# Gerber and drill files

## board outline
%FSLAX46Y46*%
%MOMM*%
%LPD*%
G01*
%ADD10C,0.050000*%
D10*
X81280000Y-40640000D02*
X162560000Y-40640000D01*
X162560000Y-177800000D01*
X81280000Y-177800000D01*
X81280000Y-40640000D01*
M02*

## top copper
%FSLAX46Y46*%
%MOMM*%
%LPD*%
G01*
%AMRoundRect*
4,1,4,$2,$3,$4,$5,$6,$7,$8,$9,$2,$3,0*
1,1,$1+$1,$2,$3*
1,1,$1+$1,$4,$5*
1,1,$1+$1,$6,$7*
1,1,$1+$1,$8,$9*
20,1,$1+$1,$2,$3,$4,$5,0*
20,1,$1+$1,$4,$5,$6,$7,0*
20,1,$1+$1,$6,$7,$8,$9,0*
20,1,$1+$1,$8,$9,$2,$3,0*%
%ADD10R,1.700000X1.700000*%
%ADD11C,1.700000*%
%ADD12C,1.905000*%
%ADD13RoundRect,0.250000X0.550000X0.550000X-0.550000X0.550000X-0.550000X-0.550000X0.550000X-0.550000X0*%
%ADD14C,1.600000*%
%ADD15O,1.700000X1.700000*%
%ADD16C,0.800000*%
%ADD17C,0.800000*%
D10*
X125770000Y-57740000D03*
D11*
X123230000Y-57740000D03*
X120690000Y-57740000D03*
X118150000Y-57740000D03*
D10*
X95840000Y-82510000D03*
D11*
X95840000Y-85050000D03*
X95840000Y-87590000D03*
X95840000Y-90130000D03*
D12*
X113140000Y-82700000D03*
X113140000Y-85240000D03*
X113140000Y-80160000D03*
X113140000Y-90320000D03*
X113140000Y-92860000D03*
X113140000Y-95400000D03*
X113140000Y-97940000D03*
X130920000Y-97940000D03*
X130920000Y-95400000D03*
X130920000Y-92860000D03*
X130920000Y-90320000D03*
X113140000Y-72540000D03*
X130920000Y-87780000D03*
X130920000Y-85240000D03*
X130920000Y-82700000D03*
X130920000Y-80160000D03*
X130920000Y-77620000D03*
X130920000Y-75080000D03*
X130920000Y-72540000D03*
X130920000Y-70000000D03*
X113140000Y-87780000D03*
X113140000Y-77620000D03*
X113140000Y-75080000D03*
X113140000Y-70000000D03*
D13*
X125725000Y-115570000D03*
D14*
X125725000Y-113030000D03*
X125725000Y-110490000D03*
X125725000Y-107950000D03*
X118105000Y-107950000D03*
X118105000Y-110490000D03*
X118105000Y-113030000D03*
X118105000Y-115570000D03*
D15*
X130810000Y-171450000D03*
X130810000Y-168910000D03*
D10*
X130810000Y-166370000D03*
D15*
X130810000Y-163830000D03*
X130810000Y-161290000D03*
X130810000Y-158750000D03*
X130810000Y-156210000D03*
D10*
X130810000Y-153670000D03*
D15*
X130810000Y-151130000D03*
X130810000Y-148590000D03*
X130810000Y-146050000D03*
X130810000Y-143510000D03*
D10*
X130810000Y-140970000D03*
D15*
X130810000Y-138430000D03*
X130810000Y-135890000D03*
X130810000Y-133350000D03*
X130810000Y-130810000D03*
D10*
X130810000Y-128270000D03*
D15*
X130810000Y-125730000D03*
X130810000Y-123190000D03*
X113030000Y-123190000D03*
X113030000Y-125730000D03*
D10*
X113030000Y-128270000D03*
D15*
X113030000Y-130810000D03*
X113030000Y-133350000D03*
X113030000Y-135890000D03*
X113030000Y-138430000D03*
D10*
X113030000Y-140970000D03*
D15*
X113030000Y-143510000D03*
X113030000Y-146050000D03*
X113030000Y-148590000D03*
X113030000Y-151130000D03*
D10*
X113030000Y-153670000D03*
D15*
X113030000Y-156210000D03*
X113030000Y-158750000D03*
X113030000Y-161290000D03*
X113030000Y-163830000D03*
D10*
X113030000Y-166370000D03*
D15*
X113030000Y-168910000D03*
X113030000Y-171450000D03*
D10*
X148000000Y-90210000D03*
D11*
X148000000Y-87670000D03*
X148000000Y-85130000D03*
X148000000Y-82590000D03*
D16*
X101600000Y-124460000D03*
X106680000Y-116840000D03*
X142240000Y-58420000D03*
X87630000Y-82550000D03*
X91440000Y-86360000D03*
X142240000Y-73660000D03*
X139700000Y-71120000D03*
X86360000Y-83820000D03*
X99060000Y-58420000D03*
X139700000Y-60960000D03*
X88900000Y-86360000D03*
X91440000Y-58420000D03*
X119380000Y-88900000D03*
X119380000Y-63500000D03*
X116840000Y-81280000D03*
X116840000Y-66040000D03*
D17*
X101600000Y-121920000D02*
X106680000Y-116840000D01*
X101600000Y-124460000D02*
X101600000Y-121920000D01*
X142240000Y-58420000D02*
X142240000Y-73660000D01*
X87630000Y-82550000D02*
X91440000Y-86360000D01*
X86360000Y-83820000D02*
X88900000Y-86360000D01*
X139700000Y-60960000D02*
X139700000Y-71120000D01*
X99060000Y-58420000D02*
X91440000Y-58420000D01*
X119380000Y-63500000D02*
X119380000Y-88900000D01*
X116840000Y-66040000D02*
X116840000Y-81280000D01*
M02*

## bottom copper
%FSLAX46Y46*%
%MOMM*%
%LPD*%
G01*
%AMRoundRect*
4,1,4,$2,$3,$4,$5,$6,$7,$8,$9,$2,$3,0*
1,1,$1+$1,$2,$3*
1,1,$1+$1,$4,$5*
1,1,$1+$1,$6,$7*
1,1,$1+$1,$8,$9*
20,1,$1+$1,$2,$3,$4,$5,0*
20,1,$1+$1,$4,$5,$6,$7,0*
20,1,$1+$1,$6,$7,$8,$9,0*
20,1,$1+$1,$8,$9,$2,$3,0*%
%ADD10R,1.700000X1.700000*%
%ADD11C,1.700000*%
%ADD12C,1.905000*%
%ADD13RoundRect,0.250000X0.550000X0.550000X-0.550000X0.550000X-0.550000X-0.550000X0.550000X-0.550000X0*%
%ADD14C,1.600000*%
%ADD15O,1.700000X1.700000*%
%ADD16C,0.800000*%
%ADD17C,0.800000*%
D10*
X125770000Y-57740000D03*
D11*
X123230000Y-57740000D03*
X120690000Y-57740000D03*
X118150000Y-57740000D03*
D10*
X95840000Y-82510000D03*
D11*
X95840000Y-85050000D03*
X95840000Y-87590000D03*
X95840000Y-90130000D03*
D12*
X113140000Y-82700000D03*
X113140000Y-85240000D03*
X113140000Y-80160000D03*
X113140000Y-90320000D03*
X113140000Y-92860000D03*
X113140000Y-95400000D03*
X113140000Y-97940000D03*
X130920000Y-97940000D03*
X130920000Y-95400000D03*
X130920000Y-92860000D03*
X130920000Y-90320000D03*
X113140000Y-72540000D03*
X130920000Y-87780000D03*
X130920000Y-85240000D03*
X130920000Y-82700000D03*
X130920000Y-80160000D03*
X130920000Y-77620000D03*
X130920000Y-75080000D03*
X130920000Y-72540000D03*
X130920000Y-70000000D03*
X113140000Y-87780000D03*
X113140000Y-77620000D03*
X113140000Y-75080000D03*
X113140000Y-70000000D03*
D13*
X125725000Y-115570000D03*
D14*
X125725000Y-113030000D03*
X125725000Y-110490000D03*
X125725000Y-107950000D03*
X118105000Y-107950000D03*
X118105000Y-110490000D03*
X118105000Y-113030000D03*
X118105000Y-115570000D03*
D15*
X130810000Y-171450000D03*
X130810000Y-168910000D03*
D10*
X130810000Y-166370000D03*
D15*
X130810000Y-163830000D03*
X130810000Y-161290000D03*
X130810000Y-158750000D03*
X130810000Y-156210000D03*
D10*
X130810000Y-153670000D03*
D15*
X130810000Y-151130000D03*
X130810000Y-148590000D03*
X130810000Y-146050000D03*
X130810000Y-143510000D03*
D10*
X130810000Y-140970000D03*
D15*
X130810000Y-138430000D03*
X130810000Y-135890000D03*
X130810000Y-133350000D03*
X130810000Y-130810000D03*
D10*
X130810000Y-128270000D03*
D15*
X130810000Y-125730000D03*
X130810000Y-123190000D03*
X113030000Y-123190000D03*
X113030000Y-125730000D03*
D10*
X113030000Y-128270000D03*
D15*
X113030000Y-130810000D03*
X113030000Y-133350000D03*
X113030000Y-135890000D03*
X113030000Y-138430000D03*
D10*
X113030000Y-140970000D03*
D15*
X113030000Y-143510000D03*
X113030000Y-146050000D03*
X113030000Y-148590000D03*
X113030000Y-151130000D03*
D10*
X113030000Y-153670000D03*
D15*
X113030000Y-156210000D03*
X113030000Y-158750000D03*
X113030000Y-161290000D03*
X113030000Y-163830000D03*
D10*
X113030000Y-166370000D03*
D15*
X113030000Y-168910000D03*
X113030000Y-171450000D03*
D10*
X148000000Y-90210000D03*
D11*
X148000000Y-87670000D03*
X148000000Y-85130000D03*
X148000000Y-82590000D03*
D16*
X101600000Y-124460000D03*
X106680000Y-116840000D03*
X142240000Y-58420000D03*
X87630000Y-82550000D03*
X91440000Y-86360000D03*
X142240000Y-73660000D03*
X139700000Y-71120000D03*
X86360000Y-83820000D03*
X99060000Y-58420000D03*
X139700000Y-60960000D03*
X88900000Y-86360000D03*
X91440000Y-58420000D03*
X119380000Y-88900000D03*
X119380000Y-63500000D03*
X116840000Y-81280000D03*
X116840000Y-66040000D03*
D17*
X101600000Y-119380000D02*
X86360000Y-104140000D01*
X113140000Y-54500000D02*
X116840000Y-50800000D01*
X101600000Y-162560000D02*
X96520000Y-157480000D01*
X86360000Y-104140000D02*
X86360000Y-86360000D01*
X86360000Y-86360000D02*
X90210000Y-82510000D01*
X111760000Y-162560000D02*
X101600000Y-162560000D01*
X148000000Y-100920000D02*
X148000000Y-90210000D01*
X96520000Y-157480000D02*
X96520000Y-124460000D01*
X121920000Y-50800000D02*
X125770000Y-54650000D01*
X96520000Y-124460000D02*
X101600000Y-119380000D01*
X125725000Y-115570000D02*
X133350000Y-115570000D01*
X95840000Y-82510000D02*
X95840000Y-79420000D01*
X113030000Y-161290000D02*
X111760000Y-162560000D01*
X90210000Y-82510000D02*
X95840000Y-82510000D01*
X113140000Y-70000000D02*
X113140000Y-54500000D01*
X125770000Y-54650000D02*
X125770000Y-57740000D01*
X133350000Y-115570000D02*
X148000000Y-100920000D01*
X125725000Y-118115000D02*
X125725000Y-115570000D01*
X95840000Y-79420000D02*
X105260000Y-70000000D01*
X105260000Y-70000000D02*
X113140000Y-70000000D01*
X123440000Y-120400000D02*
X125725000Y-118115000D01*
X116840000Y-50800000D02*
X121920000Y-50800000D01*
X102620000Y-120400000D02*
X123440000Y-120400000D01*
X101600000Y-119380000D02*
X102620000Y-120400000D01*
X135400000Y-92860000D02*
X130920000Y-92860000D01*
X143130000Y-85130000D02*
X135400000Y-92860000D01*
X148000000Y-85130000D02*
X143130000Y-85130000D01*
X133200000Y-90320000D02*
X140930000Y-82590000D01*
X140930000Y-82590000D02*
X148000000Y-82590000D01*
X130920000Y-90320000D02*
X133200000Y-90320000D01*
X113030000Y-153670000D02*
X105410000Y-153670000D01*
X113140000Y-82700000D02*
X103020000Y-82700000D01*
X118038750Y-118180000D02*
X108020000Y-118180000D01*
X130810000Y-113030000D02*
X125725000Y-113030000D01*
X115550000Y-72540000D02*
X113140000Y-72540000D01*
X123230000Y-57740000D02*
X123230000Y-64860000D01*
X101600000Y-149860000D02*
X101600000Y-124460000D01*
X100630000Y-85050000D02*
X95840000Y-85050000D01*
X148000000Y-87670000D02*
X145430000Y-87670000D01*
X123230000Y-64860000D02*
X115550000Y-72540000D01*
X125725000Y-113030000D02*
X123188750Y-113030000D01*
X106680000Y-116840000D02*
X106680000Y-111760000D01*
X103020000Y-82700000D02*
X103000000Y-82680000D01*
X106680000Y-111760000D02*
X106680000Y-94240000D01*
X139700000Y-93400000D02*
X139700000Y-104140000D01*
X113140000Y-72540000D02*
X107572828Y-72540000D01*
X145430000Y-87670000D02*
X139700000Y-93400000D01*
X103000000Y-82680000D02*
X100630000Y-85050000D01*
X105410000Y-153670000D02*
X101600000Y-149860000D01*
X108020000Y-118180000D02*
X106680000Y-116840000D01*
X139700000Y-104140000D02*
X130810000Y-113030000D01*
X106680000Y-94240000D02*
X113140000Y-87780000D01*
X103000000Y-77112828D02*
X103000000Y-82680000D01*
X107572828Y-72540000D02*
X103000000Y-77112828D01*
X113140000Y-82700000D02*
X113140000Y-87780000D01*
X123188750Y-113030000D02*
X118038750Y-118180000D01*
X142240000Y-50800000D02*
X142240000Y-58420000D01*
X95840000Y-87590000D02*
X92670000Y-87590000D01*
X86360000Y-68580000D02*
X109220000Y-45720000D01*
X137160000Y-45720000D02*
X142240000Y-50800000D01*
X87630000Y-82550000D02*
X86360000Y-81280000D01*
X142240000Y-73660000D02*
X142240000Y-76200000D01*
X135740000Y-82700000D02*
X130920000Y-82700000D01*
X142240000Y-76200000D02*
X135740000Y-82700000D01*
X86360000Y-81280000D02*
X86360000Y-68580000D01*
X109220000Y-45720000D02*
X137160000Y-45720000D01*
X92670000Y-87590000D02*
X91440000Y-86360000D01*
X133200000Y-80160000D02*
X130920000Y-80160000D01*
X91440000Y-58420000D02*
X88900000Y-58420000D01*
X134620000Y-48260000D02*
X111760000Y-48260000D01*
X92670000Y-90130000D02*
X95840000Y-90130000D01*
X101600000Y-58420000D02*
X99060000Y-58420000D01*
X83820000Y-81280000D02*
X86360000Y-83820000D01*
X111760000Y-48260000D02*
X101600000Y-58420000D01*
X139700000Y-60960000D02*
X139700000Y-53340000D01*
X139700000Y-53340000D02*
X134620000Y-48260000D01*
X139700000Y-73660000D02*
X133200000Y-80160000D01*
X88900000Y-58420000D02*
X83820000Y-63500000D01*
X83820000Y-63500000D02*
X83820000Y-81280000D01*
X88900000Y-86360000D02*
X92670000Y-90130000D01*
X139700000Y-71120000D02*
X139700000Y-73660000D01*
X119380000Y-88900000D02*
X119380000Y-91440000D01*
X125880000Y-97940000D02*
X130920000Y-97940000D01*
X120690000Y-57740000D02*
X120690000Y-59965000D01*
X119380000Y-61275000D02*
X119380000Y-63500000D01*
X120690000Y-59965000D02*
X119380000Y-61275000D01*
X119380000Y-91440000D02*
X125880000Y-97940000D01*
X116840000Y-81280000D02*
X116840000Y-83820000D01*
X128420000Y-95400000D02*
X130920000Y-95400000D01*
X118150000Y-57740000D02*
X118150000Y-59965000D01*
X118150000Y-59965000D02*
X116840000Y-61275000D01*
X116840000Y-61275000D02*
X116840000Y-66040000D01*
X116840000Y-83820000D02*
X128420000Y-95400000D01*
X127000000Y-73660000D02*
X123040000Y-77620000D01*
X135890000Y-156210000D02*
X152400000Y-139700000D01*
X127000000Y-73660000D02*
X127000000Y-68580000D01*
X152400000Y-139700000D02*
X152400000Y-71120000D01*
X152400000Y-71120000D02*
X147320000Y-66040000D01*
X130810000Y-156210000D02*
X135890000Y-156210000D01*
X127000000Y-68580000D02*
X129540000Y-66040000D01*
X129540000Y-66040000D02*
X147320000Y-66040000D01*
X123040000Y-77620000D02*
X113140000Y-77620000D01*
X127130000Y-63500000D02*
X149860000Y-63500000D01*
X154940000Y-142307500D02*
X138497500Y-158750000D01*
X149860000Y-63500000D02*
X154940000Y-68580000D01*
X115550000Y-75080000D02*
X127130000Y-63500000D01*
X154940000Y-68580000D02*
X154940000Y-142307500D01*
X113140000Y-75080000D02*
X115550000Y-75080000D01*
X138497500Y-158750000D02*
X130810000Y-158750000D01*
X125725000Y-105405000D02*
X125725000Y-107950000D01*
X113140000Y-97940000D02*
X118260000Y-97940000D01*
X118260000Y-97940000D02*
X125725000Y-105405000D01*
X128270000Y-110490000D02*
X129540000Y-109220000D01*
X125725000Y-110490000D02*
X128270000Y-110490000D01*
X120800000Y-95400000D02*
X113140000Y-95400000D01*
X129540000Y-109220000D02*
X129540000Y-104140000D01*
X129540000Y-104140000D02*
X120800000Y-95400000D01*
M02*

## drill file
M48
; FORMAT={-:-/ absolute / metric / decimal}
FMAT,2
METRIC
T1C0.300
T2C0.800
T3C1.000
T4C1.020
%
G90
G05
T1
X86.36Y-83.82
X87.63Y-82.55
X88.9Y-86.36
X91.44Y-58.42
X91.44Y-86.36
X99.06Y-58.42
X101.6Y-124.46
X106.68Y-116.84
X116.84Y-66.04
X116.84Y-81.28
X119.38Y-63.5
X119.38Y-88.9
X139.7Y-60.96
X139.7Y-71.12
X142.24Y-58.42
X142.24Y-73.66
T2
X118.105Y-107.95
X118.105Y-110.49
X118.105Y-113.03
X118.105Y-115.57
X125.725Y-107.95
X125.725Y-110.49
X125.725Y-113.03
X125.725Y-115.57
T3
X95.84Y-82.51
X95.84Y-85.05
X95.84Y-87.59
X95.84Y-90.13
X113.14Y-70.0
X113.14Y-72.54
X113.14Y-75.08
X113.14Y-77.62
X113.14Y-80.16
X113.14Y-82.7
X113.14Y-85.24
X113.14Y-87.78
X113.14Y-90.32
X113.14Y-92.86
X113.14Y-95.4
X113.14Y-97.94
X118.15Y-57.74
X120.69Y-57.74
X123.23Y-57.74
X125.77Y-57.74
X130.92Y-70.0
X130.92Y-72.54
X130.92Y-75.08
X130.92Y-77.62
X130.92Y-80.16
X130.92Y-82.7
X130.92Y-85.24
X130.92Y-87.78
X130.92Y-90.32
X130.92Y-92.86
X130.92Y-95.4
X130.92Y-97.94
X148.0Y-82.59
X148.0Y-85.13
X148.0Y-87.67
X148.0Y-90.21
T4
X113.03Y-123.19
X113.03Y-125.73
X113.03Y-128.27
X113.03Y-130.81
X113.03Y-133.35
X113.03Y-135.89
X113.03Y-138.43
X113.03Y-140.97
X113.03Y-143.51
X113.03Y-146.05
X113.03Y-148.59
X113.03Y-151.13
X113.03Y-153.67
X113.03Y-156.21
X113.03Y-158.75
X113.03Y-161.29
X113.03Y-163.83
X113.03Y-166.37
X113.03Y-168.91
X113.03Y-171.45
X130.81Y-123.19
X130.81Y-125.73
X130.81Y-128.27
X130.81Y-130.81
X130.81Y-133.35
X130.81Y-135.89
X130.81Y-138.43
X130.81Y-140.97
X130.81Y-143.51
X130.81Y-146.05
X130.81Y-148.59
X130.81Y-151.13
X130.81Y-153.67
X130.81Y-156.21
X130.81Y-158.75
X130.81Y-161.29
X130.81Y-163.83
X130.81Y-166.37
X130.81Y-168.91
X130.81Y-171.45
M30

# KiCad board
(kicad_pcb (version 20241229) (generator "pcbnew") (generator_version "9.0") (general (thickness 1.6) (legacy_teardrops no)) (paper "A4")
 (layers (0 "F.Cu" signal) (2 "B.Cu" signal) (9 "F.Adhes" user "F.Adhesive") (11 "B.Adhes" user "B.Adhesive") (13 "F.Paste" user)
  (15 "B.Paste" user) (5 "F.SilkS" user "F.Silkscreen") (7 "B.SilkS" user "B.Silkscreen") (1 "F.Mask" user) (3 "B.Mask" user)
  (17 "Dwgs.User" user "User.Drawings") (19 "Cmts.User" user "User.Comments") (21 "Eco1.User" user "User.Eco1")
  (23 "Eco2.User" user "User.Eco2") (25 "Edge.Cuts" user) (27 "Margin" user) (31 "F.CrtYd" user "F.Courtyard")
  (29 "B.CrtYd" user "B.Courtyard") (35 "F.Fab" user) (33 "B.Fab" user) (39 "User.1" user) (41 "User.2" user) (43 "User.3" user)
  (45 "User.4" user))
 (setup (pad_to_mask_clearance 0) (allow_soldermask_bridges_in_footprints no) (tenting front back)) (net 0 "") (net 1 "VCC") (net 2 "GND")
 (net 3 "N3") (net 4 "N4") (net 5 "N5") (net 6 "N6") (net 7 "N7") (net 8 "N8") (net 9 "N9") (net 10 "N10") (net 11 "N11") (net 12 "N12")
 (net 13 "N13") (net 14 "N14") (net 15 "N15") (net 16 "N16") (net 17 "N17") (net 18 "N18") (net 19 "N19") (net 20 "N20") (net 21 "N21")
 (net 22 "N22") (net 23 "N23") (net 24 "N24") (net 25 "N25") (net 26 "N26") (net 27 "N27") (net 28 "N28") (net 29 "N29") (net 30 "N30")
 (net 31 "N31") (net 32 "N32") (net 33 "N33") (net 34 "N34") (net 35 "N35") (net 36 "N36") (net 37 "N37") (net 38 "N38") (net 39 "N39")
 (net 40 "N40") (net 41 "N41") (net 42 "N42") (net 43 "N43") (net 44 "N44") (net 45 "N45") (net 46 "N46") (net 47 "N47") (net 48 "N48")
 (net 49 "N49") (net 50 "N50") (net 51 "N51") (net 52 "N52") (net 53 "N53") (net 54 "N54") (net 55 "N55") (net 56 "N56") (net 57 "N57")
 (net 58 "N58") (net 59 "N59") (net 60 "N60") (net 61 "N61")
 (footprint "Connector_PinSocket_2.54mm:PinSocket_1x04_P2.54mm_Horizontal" (layer "F.Cu") (at 125.77 57.74 -90)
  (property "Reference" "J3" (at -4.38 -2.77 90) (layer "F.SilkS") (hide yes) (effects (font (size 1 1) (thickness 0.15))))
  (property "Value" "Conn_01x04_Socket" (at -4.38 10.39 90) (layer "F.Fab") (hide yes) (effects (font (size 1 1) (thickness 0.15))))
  (pad "1" thru_hole rect (at 0 0 270) (size 1.7 1.7) (drill 1) (layers "*.Cu" "*.Mask") (remove_unused_layers no) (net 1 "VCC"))
  (pad "2" thru_hole circle (at 0 2.54 270) (size 1.7 1.7) (drill 1) (layers "*.Cu" "*.Mask") (remove_unused_layers no) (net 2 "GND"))
  (pad "3" thru_hole circle (at 0 5.08 270) (size 1.7 1.7) (drill 1) (layers "*.Cu" "*.Mask") (remove_unused_layers no) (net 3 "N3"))
  (pad "4" thru_hole circle (at 0 7.62 270) (size 1.7 1.7) (drill 1) (layers "*.Cu" "*.Mask") (remove_unused_layers no) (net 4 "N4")))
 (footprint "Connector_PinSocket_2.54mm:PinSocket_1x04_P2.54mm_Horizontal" (layer "F.Cu") (at 95.84 82.51)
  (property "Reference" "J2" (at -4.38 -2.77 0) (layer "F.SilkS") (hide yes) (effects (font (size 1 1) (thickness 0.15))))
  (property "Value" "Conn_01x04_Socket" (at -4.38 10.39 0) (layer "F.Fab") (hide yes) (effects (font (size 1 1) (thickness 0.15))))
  (pad "1" thru_hole rect (at 0 0) (size 1.7 1.7) (drill 1) (layers "*.Cu" "*.Mask") (remove_unused_layers no) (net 1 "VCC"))
  (pad "2" thru_hole circle (at 0 2.54) (size 1.7 1.7) (drill 1) (layers "*.Cu" "*.Mask") (remove_unused_layers no) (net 2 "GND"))
  (pad "3" thru_hole circle (at 0 5.08) (size 1.7 1.7) (drill 1) (layers "*.Cu" "*.Mask") (remove_unused_layers no) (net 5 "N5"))
  (pad "4" thru_hole circle (at 0 7.62) (size 1.7 1.7) (drill 1) (layers "*.Cu" "*.Mask") (remove_unused_layers no) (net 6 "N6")))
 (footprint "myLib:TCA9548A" (layer "F.Cu") (at 121.92 73.82)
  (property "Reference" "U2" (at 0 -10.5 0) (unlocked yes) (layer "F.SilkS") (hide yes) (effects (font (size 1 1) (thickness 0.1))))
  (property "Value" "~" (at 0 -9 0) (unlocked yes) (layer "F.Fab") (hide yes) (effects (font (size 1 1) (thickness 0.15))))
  (pad "1" thru_hole circle (at -8.78 8.88) (size 1.905 1.905) (drill 1) (layers "*.Cu" "*.Mask") (remove_unused_layers no) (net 2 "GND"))
  (pad "2" thru_hole circle (at -8.78 11.42) (size 1.905 1.905) (drill 1) (layers "*.Cu" "*.Mask") (remove_unused_layers no) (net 2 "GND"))
  (pad "3" thru_hole circle (at -8.78 6.34) (size 1.905 1.905) (drill 1) (layers "*.Cu" "*.Mask") (remove_unused_layers no) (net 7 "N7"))
  (pad "4" thru_hole circle (at -8.78 16.5) (size 1.905 1.905) (drill 1) (layers "*.Cu" "*.Mask") (remove_unused_layers no) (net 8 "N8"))
  (pad "5" thru_hole circle (at -8.78 19.04) (size 1.905 1.905) (drill 1) (layers "*.Cu" "*.Mask") (remove_unused_layers no) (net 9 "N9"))
  (pad "6" thru_hole circle (at -8.78 21.58) (size 1.905 1.905) (drill 1) (layers "*.Cu" "*.Mask") (remove_unused_layers no) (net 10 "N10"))
  (pad "7" thru_hole circle (at -8.78 24.12) (size 1.905 1.905) (drill 1) (layers "*.Cu" "*.Mask") (remove_unused_layers no) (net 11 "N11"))
  (pad "8" thru_hole circle (at 9 24.12) (size 1.905 1.905) (drill 1) (layers "*.Cu" "*.Mask") (remove_unused_layers no) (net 3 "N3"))
  (pad "9" thru_hole circle (at 9 21.58) (size 1.905 1.905) (drill 1) (layers "*.Cu" "*.Mask") (remove_unused_layers no) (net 4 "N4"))
  (pad "10" thru_hole circle (at 9 19.04) (size 1.905 1.905) (drill 1) (layers "*.Cu" "*.Mask") (remove_unused_layers no) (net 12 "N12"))
  (pad "11" thru_hole circle (at 9 16.5) (size 1.905 1.905) (drill 1) (layers "*.Cu" "*.Mask") (remove_unused_layers no) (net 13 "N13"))
  (pad "12" thru_hole circle (at -8.78 -1.28) (size 1.905 1.905) (drill 1) (layers "*.Cu" "*.Mask") (remove_unused_layers no) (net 2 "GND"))
  (pad "13" thru_hole circle (at 9 13.96) (size 1.905 1.905) (drill 1) (layers "*.Cu" "*.Mask") (remove_unused_layers no) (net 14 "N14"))
  (pad "14" thru_hole circle (at 9 11.42) (size 1.905 1.905) (drill 1) (layers "*.Cu" "*.Mask") (remove_unused_layers no) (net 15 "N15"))
  (pad "15" thru_hole circle (at 9 8.88) (size 1.905 1.905) (drill 1) (layers "*.Cu" "*.Mask") (remove_unused_layers no) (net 5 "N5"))
  (pad "16" thru_hole circle (at 9 6.34) (size 1.905 1.905) (drill 1) (layers "*.Cu" "*.Mask") (remove_unused_layers no) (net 6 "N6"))
  (pad "17" thru_hole circle (at 9 3.8) (size 1.905 1.905) (drill 1) (layers "*.Cu" "*.Mask") (remove_unused_layers no) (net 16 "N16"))
  (pad "18" thru_hole circle (at 9 1.26) (size 1.905 1.905) (drill 1) (layers "*.Cu" "*.Mask") (remove_unused_layers no) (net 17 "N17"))
  (pad "19" thru_hole circle (at 9 -1.28) (size 1.905 1.905) (drill 1) (layers "*.Cu" "*.Mask") (remove_unused_layers no) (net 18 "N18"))
  (pad "20" thru_hole circle (at 9 -3.82) (size 1.905 1.905) (drill 1) (layers "*.Cu" "*.Mask") (remove_unused_layers no) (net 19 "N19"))
  (pad "21" thru_hole circle (at -8.78 13.96) (size 1.905 1.905) (drill 1) (layers "*.Cu" "*.Mask") (remove_unused_layers no) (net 2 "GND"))
  (pad "22" thru_hole circle (at -8.78 3.8) (size 1.905 1.905) (drill 1) (layers "*.Cu" "*.Mask") (remove_unused_layers no) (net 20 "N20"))
  (pad "23" thru_hole circle (at -8.78 1.26) (size 1.905 1.905) (drill 1) (layers "*.Cu" "*.Mask") (remove_unused_layers no) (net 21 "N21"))
  (pad "24" thru_hole circle (at -8.78 -3.82) (size 1.905 1.905) (drill 1) (layers "*.Cu" "*.Mask") (remove_unused_layers no) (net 1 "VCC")))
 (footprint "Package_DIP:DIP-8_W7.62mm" (layer "F.Cu") (at 125.725 115.57 180)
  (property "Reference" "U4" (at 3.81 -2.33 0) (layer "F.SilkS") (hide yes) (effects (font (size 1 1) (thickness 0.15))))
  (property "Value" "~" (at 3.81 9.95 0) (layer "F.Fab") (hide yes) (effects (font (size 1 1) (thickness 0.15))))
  (pad "1" thru_hole roundrect (at 0 0 180) (size 1.6 1.6) (drill 0.8) (layers "*.Cu" "*.Mask") (remove_unused_layers no)
   (roundrect_rratio 0.15625) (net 1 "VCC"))
  (pad "2" thru_hole circle (at 0 2.54 180) (size 1.6 1.6) (drill 0.8) (layers "*.Cu" "*.Mask") (remove_unused_layers no) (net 2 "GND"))
  (pad "3" thru_hole circle (at 0 5.08 180) (size 1.6 1.6) (drill 0.8) (layers "*.Cu" "*.Mask") (remove_unused_layers no) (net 10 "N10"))
  (pad "4" thru_hole circle (at 0 7.62 180) (size 1.6 1.6) (drill 0.8) (layers "*.Cu" "*.Mask") (remove_unused_layers no) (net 11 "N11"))
  (pad "5" thru_hole circle (at 7.62 7.62 180) (size 1.6 1.6) (drill 0.8) (layers "*.Cu" "*.Mask") (remove_unused_layers no) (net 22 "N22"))
  (pad "6" thru_hole circle (at 7.62 5.08 180) (size 1.6 1.6) (drill 0.8) (layers "*.Cu" "*.Mask") (remove_unused_layers no) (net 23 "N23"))
  (pad "7" thru_hole circle (at 7.62 2.54 180) (size 1.6 1.6) (drill 0.8) (layers "*.Cu" "*.Mask") (remove_unused_layers no) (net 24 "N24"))
  (pad "8" thru_hole circle (at 7.62 0 180) (size 1.6 1.6) (drill 0.8) (layers "*.Cu" "*.Mask") (remove_unused_layers no) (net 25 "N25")))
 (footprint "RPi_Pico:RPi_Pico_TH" (layer "F.Cu") (at 121.92 147.32 180)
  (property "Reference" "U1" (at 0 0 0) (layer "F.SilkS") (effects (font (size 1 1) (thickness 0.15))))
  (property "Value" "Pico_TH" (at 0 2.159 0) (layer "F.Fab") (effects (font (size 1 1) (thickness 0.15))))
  (pad "1" thru_hole oval (at -8.89 -24.13 180) (size 1.7 1.7) (drill 1.02) (layers "*.Cu" "*.Mask") (remove_unused_layers no)
   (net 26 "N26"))
  (pad "2" thru_hole oval (at -8.89 -21.59 180) (size 1.7 1.7) (drill 1.02) (layers "*.Cu" "*.Mask") (remove_unused_layers no)
   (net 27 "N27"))
  (pad "3" thru_hole rect (at -8.89 -19.05 180) (size 1.7 1.7) (drill 1.02) (layers "*.Cu" "*.Mask") (remove_unused_layers no)
   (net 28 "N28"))
  (pad "4" thru_hole oval (at -8.89 -16.51 180) (size 1.7 1.7) (drill 1.02) (layers "*.Cu" "*.Mask") (remove_unused_layers no)
   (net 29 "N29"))
  (pad "5" thru_hole oval (at -8.89 -13.97 180) (size 1.7 1.7) (drill 1.02) (layers "*.Cu" "*.Mask") (remove_unused_layers no)
   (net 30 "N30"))
  (pad "6" thru_hole oval (at -8.89 -11.43 180) (size 1.7 1.7) (drill 1.02) (layers "*.Cu" "*.Mask") (remove_unused_layers no)
   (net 21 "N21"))
  (pad "7" thru_hole oval (at -8.89 -8.89 180) (size 1.7 1.7) (drill 1.02) (layers "*.Cu" "*.Mask") (remove_unused_layers no) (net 20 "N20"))
  (pad "8" thru_hole rect (at -8.89 -6.35 180) (size 1.7 1.7) (drill 1.02) (layers "*.Cu" "*.Mask") (remove_unused_layers no) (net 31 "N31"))
  (pad "9" thru_hole oval (at -8.89 -3.81 180) (size 1.7 1.7) (drill 1.02) (layers "*.Cu" "*.Mask") (remove_unused_layers no) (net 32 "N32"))
  (pad "10" thru_hole oval (at -8.89 -1.27 180) (size 1.7 1.7) (drill 1.02) (layers "*.Cu" "*.Mask") (remove_unused_layers no)
   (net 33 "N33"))
  (pad "11" thru_hole oval (at -8.89 1.27 180) (size 1.7 1.7) (drill 1.02) (layers "*.Cu" "*.Mask") (remove_unused_layers no) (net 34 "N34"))
  (pad "12" thru_hole oval (at -8.89 3.81 180) (size 1.7 1.7) (drill 1.02) (layers "*.Cu" "*.Mask") (remove_unused_layers no) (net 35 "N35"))
  (pad "13" thru_hole rect (at -8.89 6.35 180) (size 1.7 1.7) (drill 1.02) (layers "*.Cu" "*.Mask") (remove_unused_layers no) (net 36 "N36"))
  (pad "14" thru_hole oval (at -8.89 8.89 180) (size 1.7 1.7) (drill 1.02) (layers "*.Cu" "*.Mask") (remove_unused_layers no) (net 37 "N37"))
  (pad "15" thru_hole oval (at -8.89 11.43 180) (size 1.7 1.7) (drill 1.02) (layers "*.Cu" "*.Mask") (remove_unused_layers no)
   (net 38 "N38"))
  (pad "16" thru_hole oval (at -8.89 13.97 180) (size 1.7 1.7) (drill 1.02) (layers "*.Cu" "*.Mask") (remove_unused_layers no)
   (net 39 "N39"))
  (pad "17" thru_hole oval (at -8.89 16.51 180) (size 1.7 1.7) (drill 1.02) (layers "*.Cu" "*.Mask") (remove_unused_layers no)
   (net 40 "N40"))
  (pad "18" thru_hole rect (at -8.89 19.05 180) (size 1.7 1.7) (drill 1.02) (layers "*.Cu" "*.Mask") (remove_unused_layers no)
   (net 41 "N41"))
  (pad "19" thru_hole oval (at -8.89 21.59 180) (size 1.7 1.7) (drill 1.02) (layers "*.Cu" "*.Mask") (remove_unused_layers no)
   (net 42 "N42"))
  (pad "20" thru_hole oval (at -8.89 24.13 180) (size 1.7 1.7) (drill 1.02) (layers "*.Cu" "*.Mask") (remove_unused_layers no)
   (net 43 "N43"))
  (pad "21" thru_hole oval (at 8.89 24.13 180) (size 1.7 1.7) (drill 1.02) (layers "*.Cu" "*.Mask") (remove_unused_layers no) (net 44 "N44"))
  (pad "22" thru_hole oval (at 8.89 21.59 180) (size 1.7 1.7) (drill 1.02) (layers "*.Cu" "*.Mask") (remove_unused_layers no) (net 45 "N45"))
  (pad "23" thru_hole rect (at 8.89 19.05 180) (size 1.7 1.7) (drill 1.02) (layers "*.Cu" "*.Mask") (remove_unused_layers no) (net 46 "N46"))
  (pad "24" thru_hole oval (at 8.89 16.51 180) (size 1.7 1.7) (drill 1.02) (layers "*.Cu" "*.Mask") (remove_unused_layers no) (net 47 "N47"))
  (pad "25" thru_hole oval (at 8.89 13.97 180) (size 1.7 1.7) (drill 1.02) (layers "*.Cu" "*.Mask") (remove_unused_layers no) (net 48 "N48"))
  (pad "26" thru_hole oval (at 8.89 11.43 180) (size 1.7 1.7) (drill 1.02) (layers "*.Cu" "*.Mask") (remove_unused_layers no) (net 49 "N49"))
  (pad "27" thru_hole oval (at 8.89 8.89 180) (size 1.7 1.7) (drill 1.02) (layers "*.Cu" "*.Mask") (remove_unused_layers no) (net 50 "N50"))
  (pad "28" thru_hole rect (at 8.89 6.35 180) (size 1.7 1.7) (drill 1.02) (layers "*.Cu" "*.Mask") (remove_unused_layers no) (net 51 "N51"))
  (pad "29" thru_hole oval (at 8.89 3.81 180) (size 1.7 1.7) (drill 1.02) (layers "*.Cu" "*.Mask") (remove_unused_layers no) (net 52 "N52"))
  (pad "30" thru_hole oval (at 8.89 1.27 180) (size 1.7 1.7) (drill 1.02) (layers "*.Cu" "*.Mask") (remove_unused_layers no) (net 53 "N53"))
  (pad "31" thru_hole oval (at 8.89 -1.27 180) (size 1.7 1.7) (drill 1.02) (layers "*.Cu" "*.Mask") (remove_unused_layers no) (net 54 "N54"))
  (pad "32" thru_hole oval (at 8.89 -3.81 180) (size 1.7 1.7) (drill 1.02) (layers "*.Cu" "*.Mask") (remove_unused_layers no) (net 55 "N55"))
  (pad "33" thru_hole rect (at 8.89 -6.35 180) (size 1.7 1.7) (drill 1.02) (layers "*.Cu" "*.Mask") (remove_unused_layers no) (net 2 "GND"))
  (pad "34" thru_hole oval (at 8.89 -8.89 180) (size 1.7 1.7) (drill 1.02) (layers "*.Cu" "*.Mask") (remove_unused_layers no) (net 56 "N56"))
  (pad "35" thru_hole oval (at 8.89 -11.43 180) (size 1.7 1.7) (drill 1.02) (layers "*.Cu" "*.Mask") (remove_unused_layers no)
   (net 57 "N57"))
  (pad "36" thru_hole oval (at 8.89 -13.97 180) (size 1.7 1.7) (drill 1.02) (layers "*.Cu" "*.Mask") (remove_unused_layers no) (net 1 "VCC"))
  (pad "37" thru_hole oval (at 8.89 -16.51 180) (size 1.7 1.7) (drill 1.02) (layers "*.Cu" "*.Mask") (remove_unused_layers no)
   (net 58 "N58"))
  (pad "38" thru_hole rect (at 8.89 -19.05 180) (size 1.7 1.7) (drill 1.02) (layers "*.Cu" "*.Mask") (remove_unused_layers no)
   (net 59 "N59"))
  (pad "39" thru_hole oval (at 8.89 -21.59 180) (size 1.7 1.7) (drill 1.02) (layers "*.Cu" "*.Mask") (remove_unused_layers no)
   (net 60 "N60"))
  (pad "40" thru_hole oval (at 8.89 -24.13 180) (size 1.7 1.7) (drill 1.02) (layers "*.Cu" "*.Mask") (remove_unused_layers no)
   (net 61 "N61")))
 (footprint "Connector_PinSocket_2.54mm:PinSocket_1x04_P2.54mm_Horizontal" (layer "F.Cu") (at 148 90.21 180)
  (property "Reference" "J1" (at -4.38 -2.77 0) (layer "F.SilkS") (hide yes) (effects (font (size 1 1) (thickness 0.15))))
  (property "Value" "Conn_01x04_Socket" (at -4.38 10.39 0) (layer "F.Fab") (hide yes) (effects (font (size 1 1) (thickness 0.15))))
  (pad "1" thru_hole rect (at 0 0 180) (size 1.7 1.7) (drill 1) (layers "*.Cu" "*.Mask") (remove_unused_layers no) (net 1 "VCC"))
  (pad "2" thru_hole circle (at 0 2.54 180) (size 1.7 1.7) (drill 1) (layers "*.Cu" "*.Mask") (remove_unused_layers no) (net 2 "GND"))
  (pad "3" thru_hole circle (at 0 5.08 180) (size 1.7 1.7) (drill 1) (layers "*.Cu" "*.Mask") (remove_unused_layers no) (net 12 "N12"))
  (pad "4" thru_hole circle (at 0 7.62 180) (size 1.7 1.7) (drill 1) (layers "*.Cu" "*.Mask") (remove_unused_layers no) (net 13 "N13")))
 (gr_rect (start 81.28 40.64) (end 162.56 177.8) (stroke (width 0.05) (type default)) (fill no) (layer "Edge.Cuts"))
 (segment (start 101.6 119.38) (end 86.36 104.14) (width 0.8) (layer "B.Cu") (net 1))
 (segment (start 113.14 54.5) (end 116.84 50.8) (width 0.8) (layer "B.Cu") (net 1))
 (segment (start 101.6 162.56) (end 96.52 157.48) (width 0.8) (layer "B.Cu") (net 1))
 (segment (start 86.36 104.14) (end 86.36 86.36) (width 0.8) (layer "B.Cu") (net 1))
 (segment (start 86.36 86.36) (end 90.21 82.51) (width 0.8) (layer "B.Cu") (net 1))
 (segment (start 111.76 162.56) (end 101.6 162.56) (width 0.8) (layer "B.Cu") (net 1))
 (segment (start 148 100.92) (end 148 90.21) (width 0.8) (layer "B.Cu") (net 1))
 (segment (start 96.52 157.48) (end 96.52 124.46) (width 0.8) (layer "B.Cu") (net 1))
 (segment (start 121.92 50.8) (end 125.77 54.65) (width 0.8) (layer "B.Cu") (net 1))
 (segment (start 96.52 124.46) (end 101.6 119.38) (width 0.8) (layer "B.Cu") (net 1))
 (segment (start 125.725 115.57) (end 133.35 115.57) (width 0.8) (layer "B.Cu") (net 1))
 (segment (start 95.84 82.51) (end 95.84 79.42) (width 0.8) (layer "B.Cu") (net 1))
 (segment (start 113.03 161.29) (end 111.76 162.56) (width 0.8) (layer "B.Cu") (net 1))
 (segment (start 90.21 82.51) (end 95.84 82.51) (width 0.8) (layer "B.Cu") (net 1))
 (segment (start 113.14 70) (end 113.14 54.5) (width 0.8) (layer "B.Cu") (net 1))
 (segment (start 125.77 54.65) (end 125.77 57.74) (width 0.8) (layer "B.Cu") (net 1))
 (segment (start 133.35 115.57) (end 148 100.92) (width 0.8) (layer "B.Cu") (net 1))
 (segment (start 125.725 118.115) (end 125.725 115.57) (width 0.8) (layer "B.Cu") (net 1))
 (segment (start 95.84 79.42) (end 105.26 70) (width 0.8) (layer "B.Cu") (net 1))
 (segment (start 105.26 70) (end 113.14 70) (width 0.8) (layer "B.Cu") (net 1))
 (segment (start 123.44 120.4) (end 125.725 118.115) (width 0.8) (layer "B.Cu") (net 1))
 (segment (start 116.84 50.8) (end 121.92 50.8) (width 0.8) (layer "B.Cu") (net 1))
 (segment (start 102.62 120.4) (end 123.44 120.4) (width 0.8) (layer "B.Cu") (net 1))
 (segment (start 101.6 119.38) (end 102.62 120.4) (width 0.8) (layer "B.Cu") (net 1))
 (segment (start 135.4 92.86) (end 130.92 92.86) (width 0.8) (layer "B.Cu") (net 12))
 (segment (start 143.13 85.13) (end 135.4 92.86) (width 0.8) (layer "B.Cu") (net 12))
 (segment (start 148 85.13) (end 143.13 85.13) (width 0.8) (layer "B.Cu") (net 12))
 (segment (start 133.2 90.32) (end 140.93 82.59) (width 0.8) (layer "B.Cu") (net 13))
 (segment (start 140.93 82.59) (end 148 82.59) (width 0.8) (layer "B.Cu") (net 13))
 (segment (start 130.92 90.32) (end 133.2 90.32) (width 0.8) (layer "B.Cu") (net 13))
 (segment (start 101.6 121.92) (end 106.68 116.84) (width 0.8) (layer "F.Cu") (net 2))
 (segment (start 101.6 124.46) (end 101.6 121.92) (width 0.8) (layer "F.Cu") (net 2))
 (via (at 101.6 124.46) (size 0.8) (drill 0.3) (layers "F.Cu" "B.Cu") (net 2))
 (via (at 106.68 116.84) (size 0.8) (drill 0.3) (layers "F.Cu" "B.Cu") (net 2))
 (segment (start 113.03 153.67) (end 105.41 153.67) (width 0.8) (layer "B.Cu") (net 2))
 (segment (start 113.14 82.7) (end 103.02 82.7) (width 0.8) (layer "B.Cu") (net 2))
 (segment (start 118.03875 118.18) (end 108.02 118.18) (width 0.8) (layer "B.Cu") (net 2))
 (segment (start 130.81 113.03) (end 125.725 113.03) (width 0.8) (layer "B.Cu") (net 2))
 (segment (start 115.55 72.54) (end 113.14 72.54) (width 0.8) (layer "B.Cu") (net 2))
 (segment (start 123.23 57.74) (end 123.23 64.86) (width 0.8) (layer "B.Cu") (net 2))
 (segment (start 101.6 149.86) (end 101.6 124.46) (width 0.8) (layer "B.Cu") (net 2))
 (segment (start 100.63 85.05) (end 95.84 85.05) (width 0.8) (layer "B.Cu") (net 2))
 (segment (start 148 87.67) (end 145.43 87.67) (width 0.8) (layer "B.Cu") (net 2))
 (segment (start 123.23 64.86) (end 115.55 72.54) (width 0.8) (layer "B.Cu") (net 2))
 (segment (start 125.725 113.03) (end 123.18875 113.03) (width 0.8) (layer "B.Cu") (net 2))
 (segment (start 106.68 116.84) (end 106.68 111.76) (width 0.8) (layer "B.Cu") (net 2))
 (segment (start 103.02 82.7) (end 103 82.68) (width 0.8) (layer "B.Cu") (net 2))
 (segment (start 106.68 111.76) (end 106.68 94.24) (width 0.8) (layer "B.Cu") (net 2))
 (segment (start 139.7 93.4) (end 139.7 104.14) (width 0.8) (layer "B.Cu") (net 2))
 (segment (start 113.14 72.54) (end 107.572828 72.54) (width 0.8) (layer "B.Cu") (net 2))
 (segment (start 145.43 87.67) (end 139.7 93.4) (width 0.8) (layer "B.Cu") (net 2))
 (segment (start 103 82.68) (end 100.63 85.05) (width 0.8) (layer "B.Cu") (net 2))
 (segment (start 105.41 153.67) (end 101.6 149.86) (width 0.8) (layer "B.Cu") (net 2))
 (segment (start 108.02 118.18) (end 106.68 116.84) (width 0.8) (layer "B.Cu") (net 2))
 (segment (start 139.7 104.14) (end 130.81 113.03) (width 0.8) (layer "B.Cu") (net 2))
 (segment (start 106.68 94.24) (end 113.14 87.78) (width 0.8) (layer "B.Cu") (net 2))
 (segment (start 103 77.112828) (end 103 82.68) (width 0.8) (layer "B.Cu") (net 2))
 (segment (start 107.572828 72.54) (end 103 77.112828) (width 0.8) (layer "B.Cu") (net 2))
 (segment (start 113.14 82.7) (end 113.14 87.78) (width 0.8) (layer "B.Cu") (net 2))
 (segment (start 123.18875 113.03) (end 118.03875 118.18) (width 0.8) (layer "B.Cu") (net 2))
 (segment (start 142.24 58.42) (end 142.24 73.66) (width 0.8) (layer "F.Cu") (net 5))
 (segment (start 87.63 82.55) (end 91.44 86.36) (width 0.8) (layer "F.Cu") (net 5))
 (via (at 142.24 58.42) (size 0.8) (drill 0.3) (layers "F.Cu" "B.Cu") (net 5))
 (via (at 87.63 82.55) (size 0.8) (drill 0.3) (layers "F.Cu" "B.Cu") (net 5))
 (via (at 91.44 86.36) (size 0.8) (drill 0.3) (layers "F.Cu" "B.Cu") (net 5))
 (via (at 142.24 73.66) (size 0.8) (drill 0.3) (layers "F.Cu" "B.Cu") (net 5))
 (segment (start 142.24 50.8) (end 142.24 58.42) (width 0.8) (layer "B.Cu") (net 5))
 (segment (start 95.84 87.59) (end 92.67 87.59) (width 0.8) (layer "B.Cu") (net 5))
 (segment (start 86.36 68.58) (end 109.22 45.72) (width 0.8) (layer "B.Cu") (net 5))
 (segment (start 137.16 45.72) (end 142.24 50.8) (width 0.8) (layer "B.Cu") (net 5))
 (segment (start 87.63 82.55) (end 86.36 81.28) (width 0.8) (layer "B.Cu") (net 5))
 (segment (start 142.24 73.66) (end 142.24 76.2) (width 0.8) (layer "B.Cu") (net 5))
 (segment (start 135.74 82.7) (end 130.92 82.7) (width 0.8) (layer "B.Cu") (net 5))
 (segment (start 142.24 76.2) (end 135.74 82.7) (width 0.8) (layer "B.Cu") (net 5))
 (segment (start 86.36 81.28) (end 86.36 68.58) (width 0.8) (layer "B.Cu") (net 5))
 (segment (start 109.22 45.72) (end 137.16 45.72) (width 0.8) (layer "B.Cu") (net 5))
 (segment (start 92.67 87.59) (end 91.44 86.36) (width 0.8) (layer "B.Cu") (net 5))
 (segment (start 86.36 83.82) (end 88.9 86.36) (width 0.8) (layer "F.Cu") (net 6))
 (segment (start 139.7 60.96) (end 139.7 71.12) (width 0.8) (layer "F.Cu") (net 6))
 (segment (start 99.06 58.42) (end 91.44 58.42) (width 0.8) (layer "F.Cu") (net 6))
 (via (at 139.7 71.12) (size 0.8) (drill 0.3) (layers "F.Cu" "B.Cu") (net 6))
 (via (at 86.36 83.82) (size 0.8) (drill 0.3) (layers "F.Cu" "B.Cu") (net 6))
 (via (at 99.06 58.42) (size 0.8) (drill 0.3) (layers "F.Cu" "B.Cu") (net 6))
 (via (at 139.7 60.96) (size 0.8) (drill 0.3) (layers "F.Cu" "B.Cu") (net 6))
 (via (at 88.9 86.36) (size 0.8) (drill 0.3) (layers "F.Cu" "B.Cu") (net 6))
 (via (at 91.44 58.42) (size 0.8) (drill 0.3) (layers "F.Cu" "B.Cu") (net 6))
 (segment (start 133.2 80.16) (end 130.92 80.16) (width 0.8) (layer "B.Cu") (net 6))
 (segment (start 91.44 58.42) (end 88.9 58.42) (width 0.8) (layer "B.Cu") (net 6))
 (segment (start 134.62 48.26) (end 111.76 48.26) (width 0.8) (layer "B.Cu") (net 6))
 (segment (start 92.67 90.13) (end 95.84 90.13) (width 0.8) (layer "B.Cu") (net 6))
 (segment (start 101.6 58.42) (end 99.06 58.42) (width 0.8) (layer "B.Cu") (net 6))
 (segment (start 83.82 81.28) (end 86.36 83.82) (width 0.8) (layer "B.Cu") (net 6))
 (segment (start 111.76 48.26) (end 101.6 58.42) (width 0.8) (layer "B.Cu") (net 6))
 (segment (start 139.7 60.96) (end 139.7 53.34) (width 0.8) (layer "B.Cu") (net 6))
 (segment (start 139.7 53.34) (end 134.62 48.26) (width 0.8) (layer "B.Cu") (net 6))
 (segment (start 139.7 73.66) (end 133.2 80.16) (width 0.8) (layer "B.Cu") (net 6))
 (segment (start 88.9 58.42) (end 83.82 63.5) (width 0.8) (layer "B.Cu") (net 6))
 (segment (start 83.82 63.5) (end 83.82 81.28) (width 0.8) (layer "B.Cu") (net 6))
 (segment (start 88.9 86.36) (end 92.67 90.13) (width 0.8) (layer "B.Cu") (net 6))
 (segment (start 139.7 71.12) (end 139.7 73.66) (width 0.8) (layer "B.Cu") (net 6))
 (segment (start 119.38 63.5) (end 119.38 88.9) (width 0.8) (layer "F.Cu") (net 3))
 (via (at 119.38 88.9) (size 0.8) (drill 0.3) (layers "F.Cu" "B.Cu") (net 3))
 (via (at 119.38 63.5) (size 0.8) (drill 0.3) (layers "F.Cu" "B.Cu") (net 3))
 (segment (start 119.38 88.9) (end 119.38 91.44) (width 0.8) (layer "B.Cu") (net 3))
 (segment (start 125.88 97.94) (end 130.92 97.94) (width 0.8) (layer "B.Cu") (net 3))
 (segment (start 120.69 57.74) (end 120.69 59.965) (width 0.8) (layer "B.Cu") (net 3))
 (segment (start 119.38 61.275) (end 119.38 63.5) (width 0.8) (layer "B.Cu") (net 3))
 (segment (start 120.69 59.965) (end 119.38 61.275) (width 0.8) (layer "B.Cu") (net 3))
 (segment (start 119.38 91.44) (end 125.88 97.94) (width 0.8) (layer "B.Cu") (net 3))
 (segment (start 116.84 66.04) (end 116.84 81.28) (width 0.8) (layer "F.Cu") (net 4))
 (via (at 116.84 81.28) (size 0.8) (drill 0.3) (layers "F.Cu" "B.Cu") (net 4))
 (via (at 116.84 66.04) (size 0.8) (drill 0.3) (layers "F.Cu" "B.Cu") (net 4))
 (segment (start 116.84 81.28) (end 116.84 83.82) (width 0.8) (layer "B.Cu") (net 4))
 (segment (start 128.42 95.4) (end 130.92 95.4) (width 0.8) (layer "B.Cu") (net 4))
 (segment (start 118.15 57.74) (end 118.15 59.965) (width 0.8) (layer "B.Cu") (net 4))
 (segment (start 118.15 59.965) (end 116.84 61.275) (width 0.8) (layer "B.Cu") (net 4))
 (segment (start 116.84 61.275) (end 116.84 66.04) (width 0.8) (layer "B.Cu") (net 4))
 (segment (start 116.84 83.82) (end 128.42 95.4) (width 0.8) (layer "B.Cu") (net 4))
 (segment (start 127 73.66) (end 123.04 77.62) (width 0.8) (layer "B.Cu") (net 20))
 (segment (start 135.89 156.21) (end 152.4 139.7) (width 0.8) (layer "B.Cu") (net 20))
 (segment (start 127 73.66) (end 127 68.58) (width 0.8) (layer "B.Cu") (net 20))
 (segment (start 152.4 139.7) (end 152.4 71.12) (width 0.8) (layer "B.Cu") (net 20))
 (segment (start 152.4 71.12) (end 147.32 66.04) (width 0.8) (layer "B.Cu") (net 20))
 (segment (start 130.81 156.21) (end 135.89 156.21) (width 0.8) (layer "B.Cu") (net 20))
 (segment (start 127 68.58) (end 129.54 66.04) (width 0.8) (layer "B.Cu") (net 20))
 (segment (start 129.54 66.04) (end 147.32 66.04) (width 0.8) (layer "B.Cu") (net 20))
 (segment (start 123.04 77.62) (end 113.14 77.62) (width 0.8) (layer "B.Cu") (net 20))
 (segment (start 127.13 63.5) (end 149.86 63.5) (width 0.8) (layer "B.Cu") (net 21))
 (segment (start 154.94 142.3075) (end 138.4975 158.75) (width 0.8) (layer "B.Cu") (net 21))
 (segment (start 149.86 63.5) (end 154.94 68.58) (width 0.8) (layer "B.Cu") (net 21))
 (segment (start 115.55 75.08) (end 127.13 63.5) (width 0.8) (layer "B.Cu") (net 21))
 (segment (start 154.94 68.58) (end 154.94 142.3075) (width 0.8) (layer "B.Cu") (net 21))
 (segment (start 113.14 75.08) (end 115.55 75.08) (width 0.8) (layer "B.Cu") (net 21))
 (segment (start 138.4975 158.75) (end 130.81 158.75) (width 0.8) (layer "B.Cu") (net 21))
 (segment (start 125.725 105.405) (end 125.725 107.95) (width 0.8) (layer "B.Cu") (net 11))
 (segment (start 113.14 97.94) (end 118.26 97.94) (width 0.8) (layer "B.Cu") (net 11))
 (segment (start 118.26 97.94) (end 125.725 105.405) (width 0.8) (layer "B.Cu") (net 11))
 (segment (start 128.27 110.49) (end 129.54 109.22) (width 0.8) (layer "B.Cu") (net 10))
 (segment (start 125.725 110.49) (end 128.27 110.49) (width 0.8) (layer "B.Cu") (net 10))
 (segment (start 120.8 95.4) (end 113.14 95.4) (width 0.8) (layer "B.Cu") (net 10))
 (segment (start 129.54 109.22) (end 129.54 104.14) (width 0.8) (layer "B.Cu") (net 10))
 (segment (start 129.54 104.14) (end 120.8 95.4) (width 0.8) (layer "B.Cu") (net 10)))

